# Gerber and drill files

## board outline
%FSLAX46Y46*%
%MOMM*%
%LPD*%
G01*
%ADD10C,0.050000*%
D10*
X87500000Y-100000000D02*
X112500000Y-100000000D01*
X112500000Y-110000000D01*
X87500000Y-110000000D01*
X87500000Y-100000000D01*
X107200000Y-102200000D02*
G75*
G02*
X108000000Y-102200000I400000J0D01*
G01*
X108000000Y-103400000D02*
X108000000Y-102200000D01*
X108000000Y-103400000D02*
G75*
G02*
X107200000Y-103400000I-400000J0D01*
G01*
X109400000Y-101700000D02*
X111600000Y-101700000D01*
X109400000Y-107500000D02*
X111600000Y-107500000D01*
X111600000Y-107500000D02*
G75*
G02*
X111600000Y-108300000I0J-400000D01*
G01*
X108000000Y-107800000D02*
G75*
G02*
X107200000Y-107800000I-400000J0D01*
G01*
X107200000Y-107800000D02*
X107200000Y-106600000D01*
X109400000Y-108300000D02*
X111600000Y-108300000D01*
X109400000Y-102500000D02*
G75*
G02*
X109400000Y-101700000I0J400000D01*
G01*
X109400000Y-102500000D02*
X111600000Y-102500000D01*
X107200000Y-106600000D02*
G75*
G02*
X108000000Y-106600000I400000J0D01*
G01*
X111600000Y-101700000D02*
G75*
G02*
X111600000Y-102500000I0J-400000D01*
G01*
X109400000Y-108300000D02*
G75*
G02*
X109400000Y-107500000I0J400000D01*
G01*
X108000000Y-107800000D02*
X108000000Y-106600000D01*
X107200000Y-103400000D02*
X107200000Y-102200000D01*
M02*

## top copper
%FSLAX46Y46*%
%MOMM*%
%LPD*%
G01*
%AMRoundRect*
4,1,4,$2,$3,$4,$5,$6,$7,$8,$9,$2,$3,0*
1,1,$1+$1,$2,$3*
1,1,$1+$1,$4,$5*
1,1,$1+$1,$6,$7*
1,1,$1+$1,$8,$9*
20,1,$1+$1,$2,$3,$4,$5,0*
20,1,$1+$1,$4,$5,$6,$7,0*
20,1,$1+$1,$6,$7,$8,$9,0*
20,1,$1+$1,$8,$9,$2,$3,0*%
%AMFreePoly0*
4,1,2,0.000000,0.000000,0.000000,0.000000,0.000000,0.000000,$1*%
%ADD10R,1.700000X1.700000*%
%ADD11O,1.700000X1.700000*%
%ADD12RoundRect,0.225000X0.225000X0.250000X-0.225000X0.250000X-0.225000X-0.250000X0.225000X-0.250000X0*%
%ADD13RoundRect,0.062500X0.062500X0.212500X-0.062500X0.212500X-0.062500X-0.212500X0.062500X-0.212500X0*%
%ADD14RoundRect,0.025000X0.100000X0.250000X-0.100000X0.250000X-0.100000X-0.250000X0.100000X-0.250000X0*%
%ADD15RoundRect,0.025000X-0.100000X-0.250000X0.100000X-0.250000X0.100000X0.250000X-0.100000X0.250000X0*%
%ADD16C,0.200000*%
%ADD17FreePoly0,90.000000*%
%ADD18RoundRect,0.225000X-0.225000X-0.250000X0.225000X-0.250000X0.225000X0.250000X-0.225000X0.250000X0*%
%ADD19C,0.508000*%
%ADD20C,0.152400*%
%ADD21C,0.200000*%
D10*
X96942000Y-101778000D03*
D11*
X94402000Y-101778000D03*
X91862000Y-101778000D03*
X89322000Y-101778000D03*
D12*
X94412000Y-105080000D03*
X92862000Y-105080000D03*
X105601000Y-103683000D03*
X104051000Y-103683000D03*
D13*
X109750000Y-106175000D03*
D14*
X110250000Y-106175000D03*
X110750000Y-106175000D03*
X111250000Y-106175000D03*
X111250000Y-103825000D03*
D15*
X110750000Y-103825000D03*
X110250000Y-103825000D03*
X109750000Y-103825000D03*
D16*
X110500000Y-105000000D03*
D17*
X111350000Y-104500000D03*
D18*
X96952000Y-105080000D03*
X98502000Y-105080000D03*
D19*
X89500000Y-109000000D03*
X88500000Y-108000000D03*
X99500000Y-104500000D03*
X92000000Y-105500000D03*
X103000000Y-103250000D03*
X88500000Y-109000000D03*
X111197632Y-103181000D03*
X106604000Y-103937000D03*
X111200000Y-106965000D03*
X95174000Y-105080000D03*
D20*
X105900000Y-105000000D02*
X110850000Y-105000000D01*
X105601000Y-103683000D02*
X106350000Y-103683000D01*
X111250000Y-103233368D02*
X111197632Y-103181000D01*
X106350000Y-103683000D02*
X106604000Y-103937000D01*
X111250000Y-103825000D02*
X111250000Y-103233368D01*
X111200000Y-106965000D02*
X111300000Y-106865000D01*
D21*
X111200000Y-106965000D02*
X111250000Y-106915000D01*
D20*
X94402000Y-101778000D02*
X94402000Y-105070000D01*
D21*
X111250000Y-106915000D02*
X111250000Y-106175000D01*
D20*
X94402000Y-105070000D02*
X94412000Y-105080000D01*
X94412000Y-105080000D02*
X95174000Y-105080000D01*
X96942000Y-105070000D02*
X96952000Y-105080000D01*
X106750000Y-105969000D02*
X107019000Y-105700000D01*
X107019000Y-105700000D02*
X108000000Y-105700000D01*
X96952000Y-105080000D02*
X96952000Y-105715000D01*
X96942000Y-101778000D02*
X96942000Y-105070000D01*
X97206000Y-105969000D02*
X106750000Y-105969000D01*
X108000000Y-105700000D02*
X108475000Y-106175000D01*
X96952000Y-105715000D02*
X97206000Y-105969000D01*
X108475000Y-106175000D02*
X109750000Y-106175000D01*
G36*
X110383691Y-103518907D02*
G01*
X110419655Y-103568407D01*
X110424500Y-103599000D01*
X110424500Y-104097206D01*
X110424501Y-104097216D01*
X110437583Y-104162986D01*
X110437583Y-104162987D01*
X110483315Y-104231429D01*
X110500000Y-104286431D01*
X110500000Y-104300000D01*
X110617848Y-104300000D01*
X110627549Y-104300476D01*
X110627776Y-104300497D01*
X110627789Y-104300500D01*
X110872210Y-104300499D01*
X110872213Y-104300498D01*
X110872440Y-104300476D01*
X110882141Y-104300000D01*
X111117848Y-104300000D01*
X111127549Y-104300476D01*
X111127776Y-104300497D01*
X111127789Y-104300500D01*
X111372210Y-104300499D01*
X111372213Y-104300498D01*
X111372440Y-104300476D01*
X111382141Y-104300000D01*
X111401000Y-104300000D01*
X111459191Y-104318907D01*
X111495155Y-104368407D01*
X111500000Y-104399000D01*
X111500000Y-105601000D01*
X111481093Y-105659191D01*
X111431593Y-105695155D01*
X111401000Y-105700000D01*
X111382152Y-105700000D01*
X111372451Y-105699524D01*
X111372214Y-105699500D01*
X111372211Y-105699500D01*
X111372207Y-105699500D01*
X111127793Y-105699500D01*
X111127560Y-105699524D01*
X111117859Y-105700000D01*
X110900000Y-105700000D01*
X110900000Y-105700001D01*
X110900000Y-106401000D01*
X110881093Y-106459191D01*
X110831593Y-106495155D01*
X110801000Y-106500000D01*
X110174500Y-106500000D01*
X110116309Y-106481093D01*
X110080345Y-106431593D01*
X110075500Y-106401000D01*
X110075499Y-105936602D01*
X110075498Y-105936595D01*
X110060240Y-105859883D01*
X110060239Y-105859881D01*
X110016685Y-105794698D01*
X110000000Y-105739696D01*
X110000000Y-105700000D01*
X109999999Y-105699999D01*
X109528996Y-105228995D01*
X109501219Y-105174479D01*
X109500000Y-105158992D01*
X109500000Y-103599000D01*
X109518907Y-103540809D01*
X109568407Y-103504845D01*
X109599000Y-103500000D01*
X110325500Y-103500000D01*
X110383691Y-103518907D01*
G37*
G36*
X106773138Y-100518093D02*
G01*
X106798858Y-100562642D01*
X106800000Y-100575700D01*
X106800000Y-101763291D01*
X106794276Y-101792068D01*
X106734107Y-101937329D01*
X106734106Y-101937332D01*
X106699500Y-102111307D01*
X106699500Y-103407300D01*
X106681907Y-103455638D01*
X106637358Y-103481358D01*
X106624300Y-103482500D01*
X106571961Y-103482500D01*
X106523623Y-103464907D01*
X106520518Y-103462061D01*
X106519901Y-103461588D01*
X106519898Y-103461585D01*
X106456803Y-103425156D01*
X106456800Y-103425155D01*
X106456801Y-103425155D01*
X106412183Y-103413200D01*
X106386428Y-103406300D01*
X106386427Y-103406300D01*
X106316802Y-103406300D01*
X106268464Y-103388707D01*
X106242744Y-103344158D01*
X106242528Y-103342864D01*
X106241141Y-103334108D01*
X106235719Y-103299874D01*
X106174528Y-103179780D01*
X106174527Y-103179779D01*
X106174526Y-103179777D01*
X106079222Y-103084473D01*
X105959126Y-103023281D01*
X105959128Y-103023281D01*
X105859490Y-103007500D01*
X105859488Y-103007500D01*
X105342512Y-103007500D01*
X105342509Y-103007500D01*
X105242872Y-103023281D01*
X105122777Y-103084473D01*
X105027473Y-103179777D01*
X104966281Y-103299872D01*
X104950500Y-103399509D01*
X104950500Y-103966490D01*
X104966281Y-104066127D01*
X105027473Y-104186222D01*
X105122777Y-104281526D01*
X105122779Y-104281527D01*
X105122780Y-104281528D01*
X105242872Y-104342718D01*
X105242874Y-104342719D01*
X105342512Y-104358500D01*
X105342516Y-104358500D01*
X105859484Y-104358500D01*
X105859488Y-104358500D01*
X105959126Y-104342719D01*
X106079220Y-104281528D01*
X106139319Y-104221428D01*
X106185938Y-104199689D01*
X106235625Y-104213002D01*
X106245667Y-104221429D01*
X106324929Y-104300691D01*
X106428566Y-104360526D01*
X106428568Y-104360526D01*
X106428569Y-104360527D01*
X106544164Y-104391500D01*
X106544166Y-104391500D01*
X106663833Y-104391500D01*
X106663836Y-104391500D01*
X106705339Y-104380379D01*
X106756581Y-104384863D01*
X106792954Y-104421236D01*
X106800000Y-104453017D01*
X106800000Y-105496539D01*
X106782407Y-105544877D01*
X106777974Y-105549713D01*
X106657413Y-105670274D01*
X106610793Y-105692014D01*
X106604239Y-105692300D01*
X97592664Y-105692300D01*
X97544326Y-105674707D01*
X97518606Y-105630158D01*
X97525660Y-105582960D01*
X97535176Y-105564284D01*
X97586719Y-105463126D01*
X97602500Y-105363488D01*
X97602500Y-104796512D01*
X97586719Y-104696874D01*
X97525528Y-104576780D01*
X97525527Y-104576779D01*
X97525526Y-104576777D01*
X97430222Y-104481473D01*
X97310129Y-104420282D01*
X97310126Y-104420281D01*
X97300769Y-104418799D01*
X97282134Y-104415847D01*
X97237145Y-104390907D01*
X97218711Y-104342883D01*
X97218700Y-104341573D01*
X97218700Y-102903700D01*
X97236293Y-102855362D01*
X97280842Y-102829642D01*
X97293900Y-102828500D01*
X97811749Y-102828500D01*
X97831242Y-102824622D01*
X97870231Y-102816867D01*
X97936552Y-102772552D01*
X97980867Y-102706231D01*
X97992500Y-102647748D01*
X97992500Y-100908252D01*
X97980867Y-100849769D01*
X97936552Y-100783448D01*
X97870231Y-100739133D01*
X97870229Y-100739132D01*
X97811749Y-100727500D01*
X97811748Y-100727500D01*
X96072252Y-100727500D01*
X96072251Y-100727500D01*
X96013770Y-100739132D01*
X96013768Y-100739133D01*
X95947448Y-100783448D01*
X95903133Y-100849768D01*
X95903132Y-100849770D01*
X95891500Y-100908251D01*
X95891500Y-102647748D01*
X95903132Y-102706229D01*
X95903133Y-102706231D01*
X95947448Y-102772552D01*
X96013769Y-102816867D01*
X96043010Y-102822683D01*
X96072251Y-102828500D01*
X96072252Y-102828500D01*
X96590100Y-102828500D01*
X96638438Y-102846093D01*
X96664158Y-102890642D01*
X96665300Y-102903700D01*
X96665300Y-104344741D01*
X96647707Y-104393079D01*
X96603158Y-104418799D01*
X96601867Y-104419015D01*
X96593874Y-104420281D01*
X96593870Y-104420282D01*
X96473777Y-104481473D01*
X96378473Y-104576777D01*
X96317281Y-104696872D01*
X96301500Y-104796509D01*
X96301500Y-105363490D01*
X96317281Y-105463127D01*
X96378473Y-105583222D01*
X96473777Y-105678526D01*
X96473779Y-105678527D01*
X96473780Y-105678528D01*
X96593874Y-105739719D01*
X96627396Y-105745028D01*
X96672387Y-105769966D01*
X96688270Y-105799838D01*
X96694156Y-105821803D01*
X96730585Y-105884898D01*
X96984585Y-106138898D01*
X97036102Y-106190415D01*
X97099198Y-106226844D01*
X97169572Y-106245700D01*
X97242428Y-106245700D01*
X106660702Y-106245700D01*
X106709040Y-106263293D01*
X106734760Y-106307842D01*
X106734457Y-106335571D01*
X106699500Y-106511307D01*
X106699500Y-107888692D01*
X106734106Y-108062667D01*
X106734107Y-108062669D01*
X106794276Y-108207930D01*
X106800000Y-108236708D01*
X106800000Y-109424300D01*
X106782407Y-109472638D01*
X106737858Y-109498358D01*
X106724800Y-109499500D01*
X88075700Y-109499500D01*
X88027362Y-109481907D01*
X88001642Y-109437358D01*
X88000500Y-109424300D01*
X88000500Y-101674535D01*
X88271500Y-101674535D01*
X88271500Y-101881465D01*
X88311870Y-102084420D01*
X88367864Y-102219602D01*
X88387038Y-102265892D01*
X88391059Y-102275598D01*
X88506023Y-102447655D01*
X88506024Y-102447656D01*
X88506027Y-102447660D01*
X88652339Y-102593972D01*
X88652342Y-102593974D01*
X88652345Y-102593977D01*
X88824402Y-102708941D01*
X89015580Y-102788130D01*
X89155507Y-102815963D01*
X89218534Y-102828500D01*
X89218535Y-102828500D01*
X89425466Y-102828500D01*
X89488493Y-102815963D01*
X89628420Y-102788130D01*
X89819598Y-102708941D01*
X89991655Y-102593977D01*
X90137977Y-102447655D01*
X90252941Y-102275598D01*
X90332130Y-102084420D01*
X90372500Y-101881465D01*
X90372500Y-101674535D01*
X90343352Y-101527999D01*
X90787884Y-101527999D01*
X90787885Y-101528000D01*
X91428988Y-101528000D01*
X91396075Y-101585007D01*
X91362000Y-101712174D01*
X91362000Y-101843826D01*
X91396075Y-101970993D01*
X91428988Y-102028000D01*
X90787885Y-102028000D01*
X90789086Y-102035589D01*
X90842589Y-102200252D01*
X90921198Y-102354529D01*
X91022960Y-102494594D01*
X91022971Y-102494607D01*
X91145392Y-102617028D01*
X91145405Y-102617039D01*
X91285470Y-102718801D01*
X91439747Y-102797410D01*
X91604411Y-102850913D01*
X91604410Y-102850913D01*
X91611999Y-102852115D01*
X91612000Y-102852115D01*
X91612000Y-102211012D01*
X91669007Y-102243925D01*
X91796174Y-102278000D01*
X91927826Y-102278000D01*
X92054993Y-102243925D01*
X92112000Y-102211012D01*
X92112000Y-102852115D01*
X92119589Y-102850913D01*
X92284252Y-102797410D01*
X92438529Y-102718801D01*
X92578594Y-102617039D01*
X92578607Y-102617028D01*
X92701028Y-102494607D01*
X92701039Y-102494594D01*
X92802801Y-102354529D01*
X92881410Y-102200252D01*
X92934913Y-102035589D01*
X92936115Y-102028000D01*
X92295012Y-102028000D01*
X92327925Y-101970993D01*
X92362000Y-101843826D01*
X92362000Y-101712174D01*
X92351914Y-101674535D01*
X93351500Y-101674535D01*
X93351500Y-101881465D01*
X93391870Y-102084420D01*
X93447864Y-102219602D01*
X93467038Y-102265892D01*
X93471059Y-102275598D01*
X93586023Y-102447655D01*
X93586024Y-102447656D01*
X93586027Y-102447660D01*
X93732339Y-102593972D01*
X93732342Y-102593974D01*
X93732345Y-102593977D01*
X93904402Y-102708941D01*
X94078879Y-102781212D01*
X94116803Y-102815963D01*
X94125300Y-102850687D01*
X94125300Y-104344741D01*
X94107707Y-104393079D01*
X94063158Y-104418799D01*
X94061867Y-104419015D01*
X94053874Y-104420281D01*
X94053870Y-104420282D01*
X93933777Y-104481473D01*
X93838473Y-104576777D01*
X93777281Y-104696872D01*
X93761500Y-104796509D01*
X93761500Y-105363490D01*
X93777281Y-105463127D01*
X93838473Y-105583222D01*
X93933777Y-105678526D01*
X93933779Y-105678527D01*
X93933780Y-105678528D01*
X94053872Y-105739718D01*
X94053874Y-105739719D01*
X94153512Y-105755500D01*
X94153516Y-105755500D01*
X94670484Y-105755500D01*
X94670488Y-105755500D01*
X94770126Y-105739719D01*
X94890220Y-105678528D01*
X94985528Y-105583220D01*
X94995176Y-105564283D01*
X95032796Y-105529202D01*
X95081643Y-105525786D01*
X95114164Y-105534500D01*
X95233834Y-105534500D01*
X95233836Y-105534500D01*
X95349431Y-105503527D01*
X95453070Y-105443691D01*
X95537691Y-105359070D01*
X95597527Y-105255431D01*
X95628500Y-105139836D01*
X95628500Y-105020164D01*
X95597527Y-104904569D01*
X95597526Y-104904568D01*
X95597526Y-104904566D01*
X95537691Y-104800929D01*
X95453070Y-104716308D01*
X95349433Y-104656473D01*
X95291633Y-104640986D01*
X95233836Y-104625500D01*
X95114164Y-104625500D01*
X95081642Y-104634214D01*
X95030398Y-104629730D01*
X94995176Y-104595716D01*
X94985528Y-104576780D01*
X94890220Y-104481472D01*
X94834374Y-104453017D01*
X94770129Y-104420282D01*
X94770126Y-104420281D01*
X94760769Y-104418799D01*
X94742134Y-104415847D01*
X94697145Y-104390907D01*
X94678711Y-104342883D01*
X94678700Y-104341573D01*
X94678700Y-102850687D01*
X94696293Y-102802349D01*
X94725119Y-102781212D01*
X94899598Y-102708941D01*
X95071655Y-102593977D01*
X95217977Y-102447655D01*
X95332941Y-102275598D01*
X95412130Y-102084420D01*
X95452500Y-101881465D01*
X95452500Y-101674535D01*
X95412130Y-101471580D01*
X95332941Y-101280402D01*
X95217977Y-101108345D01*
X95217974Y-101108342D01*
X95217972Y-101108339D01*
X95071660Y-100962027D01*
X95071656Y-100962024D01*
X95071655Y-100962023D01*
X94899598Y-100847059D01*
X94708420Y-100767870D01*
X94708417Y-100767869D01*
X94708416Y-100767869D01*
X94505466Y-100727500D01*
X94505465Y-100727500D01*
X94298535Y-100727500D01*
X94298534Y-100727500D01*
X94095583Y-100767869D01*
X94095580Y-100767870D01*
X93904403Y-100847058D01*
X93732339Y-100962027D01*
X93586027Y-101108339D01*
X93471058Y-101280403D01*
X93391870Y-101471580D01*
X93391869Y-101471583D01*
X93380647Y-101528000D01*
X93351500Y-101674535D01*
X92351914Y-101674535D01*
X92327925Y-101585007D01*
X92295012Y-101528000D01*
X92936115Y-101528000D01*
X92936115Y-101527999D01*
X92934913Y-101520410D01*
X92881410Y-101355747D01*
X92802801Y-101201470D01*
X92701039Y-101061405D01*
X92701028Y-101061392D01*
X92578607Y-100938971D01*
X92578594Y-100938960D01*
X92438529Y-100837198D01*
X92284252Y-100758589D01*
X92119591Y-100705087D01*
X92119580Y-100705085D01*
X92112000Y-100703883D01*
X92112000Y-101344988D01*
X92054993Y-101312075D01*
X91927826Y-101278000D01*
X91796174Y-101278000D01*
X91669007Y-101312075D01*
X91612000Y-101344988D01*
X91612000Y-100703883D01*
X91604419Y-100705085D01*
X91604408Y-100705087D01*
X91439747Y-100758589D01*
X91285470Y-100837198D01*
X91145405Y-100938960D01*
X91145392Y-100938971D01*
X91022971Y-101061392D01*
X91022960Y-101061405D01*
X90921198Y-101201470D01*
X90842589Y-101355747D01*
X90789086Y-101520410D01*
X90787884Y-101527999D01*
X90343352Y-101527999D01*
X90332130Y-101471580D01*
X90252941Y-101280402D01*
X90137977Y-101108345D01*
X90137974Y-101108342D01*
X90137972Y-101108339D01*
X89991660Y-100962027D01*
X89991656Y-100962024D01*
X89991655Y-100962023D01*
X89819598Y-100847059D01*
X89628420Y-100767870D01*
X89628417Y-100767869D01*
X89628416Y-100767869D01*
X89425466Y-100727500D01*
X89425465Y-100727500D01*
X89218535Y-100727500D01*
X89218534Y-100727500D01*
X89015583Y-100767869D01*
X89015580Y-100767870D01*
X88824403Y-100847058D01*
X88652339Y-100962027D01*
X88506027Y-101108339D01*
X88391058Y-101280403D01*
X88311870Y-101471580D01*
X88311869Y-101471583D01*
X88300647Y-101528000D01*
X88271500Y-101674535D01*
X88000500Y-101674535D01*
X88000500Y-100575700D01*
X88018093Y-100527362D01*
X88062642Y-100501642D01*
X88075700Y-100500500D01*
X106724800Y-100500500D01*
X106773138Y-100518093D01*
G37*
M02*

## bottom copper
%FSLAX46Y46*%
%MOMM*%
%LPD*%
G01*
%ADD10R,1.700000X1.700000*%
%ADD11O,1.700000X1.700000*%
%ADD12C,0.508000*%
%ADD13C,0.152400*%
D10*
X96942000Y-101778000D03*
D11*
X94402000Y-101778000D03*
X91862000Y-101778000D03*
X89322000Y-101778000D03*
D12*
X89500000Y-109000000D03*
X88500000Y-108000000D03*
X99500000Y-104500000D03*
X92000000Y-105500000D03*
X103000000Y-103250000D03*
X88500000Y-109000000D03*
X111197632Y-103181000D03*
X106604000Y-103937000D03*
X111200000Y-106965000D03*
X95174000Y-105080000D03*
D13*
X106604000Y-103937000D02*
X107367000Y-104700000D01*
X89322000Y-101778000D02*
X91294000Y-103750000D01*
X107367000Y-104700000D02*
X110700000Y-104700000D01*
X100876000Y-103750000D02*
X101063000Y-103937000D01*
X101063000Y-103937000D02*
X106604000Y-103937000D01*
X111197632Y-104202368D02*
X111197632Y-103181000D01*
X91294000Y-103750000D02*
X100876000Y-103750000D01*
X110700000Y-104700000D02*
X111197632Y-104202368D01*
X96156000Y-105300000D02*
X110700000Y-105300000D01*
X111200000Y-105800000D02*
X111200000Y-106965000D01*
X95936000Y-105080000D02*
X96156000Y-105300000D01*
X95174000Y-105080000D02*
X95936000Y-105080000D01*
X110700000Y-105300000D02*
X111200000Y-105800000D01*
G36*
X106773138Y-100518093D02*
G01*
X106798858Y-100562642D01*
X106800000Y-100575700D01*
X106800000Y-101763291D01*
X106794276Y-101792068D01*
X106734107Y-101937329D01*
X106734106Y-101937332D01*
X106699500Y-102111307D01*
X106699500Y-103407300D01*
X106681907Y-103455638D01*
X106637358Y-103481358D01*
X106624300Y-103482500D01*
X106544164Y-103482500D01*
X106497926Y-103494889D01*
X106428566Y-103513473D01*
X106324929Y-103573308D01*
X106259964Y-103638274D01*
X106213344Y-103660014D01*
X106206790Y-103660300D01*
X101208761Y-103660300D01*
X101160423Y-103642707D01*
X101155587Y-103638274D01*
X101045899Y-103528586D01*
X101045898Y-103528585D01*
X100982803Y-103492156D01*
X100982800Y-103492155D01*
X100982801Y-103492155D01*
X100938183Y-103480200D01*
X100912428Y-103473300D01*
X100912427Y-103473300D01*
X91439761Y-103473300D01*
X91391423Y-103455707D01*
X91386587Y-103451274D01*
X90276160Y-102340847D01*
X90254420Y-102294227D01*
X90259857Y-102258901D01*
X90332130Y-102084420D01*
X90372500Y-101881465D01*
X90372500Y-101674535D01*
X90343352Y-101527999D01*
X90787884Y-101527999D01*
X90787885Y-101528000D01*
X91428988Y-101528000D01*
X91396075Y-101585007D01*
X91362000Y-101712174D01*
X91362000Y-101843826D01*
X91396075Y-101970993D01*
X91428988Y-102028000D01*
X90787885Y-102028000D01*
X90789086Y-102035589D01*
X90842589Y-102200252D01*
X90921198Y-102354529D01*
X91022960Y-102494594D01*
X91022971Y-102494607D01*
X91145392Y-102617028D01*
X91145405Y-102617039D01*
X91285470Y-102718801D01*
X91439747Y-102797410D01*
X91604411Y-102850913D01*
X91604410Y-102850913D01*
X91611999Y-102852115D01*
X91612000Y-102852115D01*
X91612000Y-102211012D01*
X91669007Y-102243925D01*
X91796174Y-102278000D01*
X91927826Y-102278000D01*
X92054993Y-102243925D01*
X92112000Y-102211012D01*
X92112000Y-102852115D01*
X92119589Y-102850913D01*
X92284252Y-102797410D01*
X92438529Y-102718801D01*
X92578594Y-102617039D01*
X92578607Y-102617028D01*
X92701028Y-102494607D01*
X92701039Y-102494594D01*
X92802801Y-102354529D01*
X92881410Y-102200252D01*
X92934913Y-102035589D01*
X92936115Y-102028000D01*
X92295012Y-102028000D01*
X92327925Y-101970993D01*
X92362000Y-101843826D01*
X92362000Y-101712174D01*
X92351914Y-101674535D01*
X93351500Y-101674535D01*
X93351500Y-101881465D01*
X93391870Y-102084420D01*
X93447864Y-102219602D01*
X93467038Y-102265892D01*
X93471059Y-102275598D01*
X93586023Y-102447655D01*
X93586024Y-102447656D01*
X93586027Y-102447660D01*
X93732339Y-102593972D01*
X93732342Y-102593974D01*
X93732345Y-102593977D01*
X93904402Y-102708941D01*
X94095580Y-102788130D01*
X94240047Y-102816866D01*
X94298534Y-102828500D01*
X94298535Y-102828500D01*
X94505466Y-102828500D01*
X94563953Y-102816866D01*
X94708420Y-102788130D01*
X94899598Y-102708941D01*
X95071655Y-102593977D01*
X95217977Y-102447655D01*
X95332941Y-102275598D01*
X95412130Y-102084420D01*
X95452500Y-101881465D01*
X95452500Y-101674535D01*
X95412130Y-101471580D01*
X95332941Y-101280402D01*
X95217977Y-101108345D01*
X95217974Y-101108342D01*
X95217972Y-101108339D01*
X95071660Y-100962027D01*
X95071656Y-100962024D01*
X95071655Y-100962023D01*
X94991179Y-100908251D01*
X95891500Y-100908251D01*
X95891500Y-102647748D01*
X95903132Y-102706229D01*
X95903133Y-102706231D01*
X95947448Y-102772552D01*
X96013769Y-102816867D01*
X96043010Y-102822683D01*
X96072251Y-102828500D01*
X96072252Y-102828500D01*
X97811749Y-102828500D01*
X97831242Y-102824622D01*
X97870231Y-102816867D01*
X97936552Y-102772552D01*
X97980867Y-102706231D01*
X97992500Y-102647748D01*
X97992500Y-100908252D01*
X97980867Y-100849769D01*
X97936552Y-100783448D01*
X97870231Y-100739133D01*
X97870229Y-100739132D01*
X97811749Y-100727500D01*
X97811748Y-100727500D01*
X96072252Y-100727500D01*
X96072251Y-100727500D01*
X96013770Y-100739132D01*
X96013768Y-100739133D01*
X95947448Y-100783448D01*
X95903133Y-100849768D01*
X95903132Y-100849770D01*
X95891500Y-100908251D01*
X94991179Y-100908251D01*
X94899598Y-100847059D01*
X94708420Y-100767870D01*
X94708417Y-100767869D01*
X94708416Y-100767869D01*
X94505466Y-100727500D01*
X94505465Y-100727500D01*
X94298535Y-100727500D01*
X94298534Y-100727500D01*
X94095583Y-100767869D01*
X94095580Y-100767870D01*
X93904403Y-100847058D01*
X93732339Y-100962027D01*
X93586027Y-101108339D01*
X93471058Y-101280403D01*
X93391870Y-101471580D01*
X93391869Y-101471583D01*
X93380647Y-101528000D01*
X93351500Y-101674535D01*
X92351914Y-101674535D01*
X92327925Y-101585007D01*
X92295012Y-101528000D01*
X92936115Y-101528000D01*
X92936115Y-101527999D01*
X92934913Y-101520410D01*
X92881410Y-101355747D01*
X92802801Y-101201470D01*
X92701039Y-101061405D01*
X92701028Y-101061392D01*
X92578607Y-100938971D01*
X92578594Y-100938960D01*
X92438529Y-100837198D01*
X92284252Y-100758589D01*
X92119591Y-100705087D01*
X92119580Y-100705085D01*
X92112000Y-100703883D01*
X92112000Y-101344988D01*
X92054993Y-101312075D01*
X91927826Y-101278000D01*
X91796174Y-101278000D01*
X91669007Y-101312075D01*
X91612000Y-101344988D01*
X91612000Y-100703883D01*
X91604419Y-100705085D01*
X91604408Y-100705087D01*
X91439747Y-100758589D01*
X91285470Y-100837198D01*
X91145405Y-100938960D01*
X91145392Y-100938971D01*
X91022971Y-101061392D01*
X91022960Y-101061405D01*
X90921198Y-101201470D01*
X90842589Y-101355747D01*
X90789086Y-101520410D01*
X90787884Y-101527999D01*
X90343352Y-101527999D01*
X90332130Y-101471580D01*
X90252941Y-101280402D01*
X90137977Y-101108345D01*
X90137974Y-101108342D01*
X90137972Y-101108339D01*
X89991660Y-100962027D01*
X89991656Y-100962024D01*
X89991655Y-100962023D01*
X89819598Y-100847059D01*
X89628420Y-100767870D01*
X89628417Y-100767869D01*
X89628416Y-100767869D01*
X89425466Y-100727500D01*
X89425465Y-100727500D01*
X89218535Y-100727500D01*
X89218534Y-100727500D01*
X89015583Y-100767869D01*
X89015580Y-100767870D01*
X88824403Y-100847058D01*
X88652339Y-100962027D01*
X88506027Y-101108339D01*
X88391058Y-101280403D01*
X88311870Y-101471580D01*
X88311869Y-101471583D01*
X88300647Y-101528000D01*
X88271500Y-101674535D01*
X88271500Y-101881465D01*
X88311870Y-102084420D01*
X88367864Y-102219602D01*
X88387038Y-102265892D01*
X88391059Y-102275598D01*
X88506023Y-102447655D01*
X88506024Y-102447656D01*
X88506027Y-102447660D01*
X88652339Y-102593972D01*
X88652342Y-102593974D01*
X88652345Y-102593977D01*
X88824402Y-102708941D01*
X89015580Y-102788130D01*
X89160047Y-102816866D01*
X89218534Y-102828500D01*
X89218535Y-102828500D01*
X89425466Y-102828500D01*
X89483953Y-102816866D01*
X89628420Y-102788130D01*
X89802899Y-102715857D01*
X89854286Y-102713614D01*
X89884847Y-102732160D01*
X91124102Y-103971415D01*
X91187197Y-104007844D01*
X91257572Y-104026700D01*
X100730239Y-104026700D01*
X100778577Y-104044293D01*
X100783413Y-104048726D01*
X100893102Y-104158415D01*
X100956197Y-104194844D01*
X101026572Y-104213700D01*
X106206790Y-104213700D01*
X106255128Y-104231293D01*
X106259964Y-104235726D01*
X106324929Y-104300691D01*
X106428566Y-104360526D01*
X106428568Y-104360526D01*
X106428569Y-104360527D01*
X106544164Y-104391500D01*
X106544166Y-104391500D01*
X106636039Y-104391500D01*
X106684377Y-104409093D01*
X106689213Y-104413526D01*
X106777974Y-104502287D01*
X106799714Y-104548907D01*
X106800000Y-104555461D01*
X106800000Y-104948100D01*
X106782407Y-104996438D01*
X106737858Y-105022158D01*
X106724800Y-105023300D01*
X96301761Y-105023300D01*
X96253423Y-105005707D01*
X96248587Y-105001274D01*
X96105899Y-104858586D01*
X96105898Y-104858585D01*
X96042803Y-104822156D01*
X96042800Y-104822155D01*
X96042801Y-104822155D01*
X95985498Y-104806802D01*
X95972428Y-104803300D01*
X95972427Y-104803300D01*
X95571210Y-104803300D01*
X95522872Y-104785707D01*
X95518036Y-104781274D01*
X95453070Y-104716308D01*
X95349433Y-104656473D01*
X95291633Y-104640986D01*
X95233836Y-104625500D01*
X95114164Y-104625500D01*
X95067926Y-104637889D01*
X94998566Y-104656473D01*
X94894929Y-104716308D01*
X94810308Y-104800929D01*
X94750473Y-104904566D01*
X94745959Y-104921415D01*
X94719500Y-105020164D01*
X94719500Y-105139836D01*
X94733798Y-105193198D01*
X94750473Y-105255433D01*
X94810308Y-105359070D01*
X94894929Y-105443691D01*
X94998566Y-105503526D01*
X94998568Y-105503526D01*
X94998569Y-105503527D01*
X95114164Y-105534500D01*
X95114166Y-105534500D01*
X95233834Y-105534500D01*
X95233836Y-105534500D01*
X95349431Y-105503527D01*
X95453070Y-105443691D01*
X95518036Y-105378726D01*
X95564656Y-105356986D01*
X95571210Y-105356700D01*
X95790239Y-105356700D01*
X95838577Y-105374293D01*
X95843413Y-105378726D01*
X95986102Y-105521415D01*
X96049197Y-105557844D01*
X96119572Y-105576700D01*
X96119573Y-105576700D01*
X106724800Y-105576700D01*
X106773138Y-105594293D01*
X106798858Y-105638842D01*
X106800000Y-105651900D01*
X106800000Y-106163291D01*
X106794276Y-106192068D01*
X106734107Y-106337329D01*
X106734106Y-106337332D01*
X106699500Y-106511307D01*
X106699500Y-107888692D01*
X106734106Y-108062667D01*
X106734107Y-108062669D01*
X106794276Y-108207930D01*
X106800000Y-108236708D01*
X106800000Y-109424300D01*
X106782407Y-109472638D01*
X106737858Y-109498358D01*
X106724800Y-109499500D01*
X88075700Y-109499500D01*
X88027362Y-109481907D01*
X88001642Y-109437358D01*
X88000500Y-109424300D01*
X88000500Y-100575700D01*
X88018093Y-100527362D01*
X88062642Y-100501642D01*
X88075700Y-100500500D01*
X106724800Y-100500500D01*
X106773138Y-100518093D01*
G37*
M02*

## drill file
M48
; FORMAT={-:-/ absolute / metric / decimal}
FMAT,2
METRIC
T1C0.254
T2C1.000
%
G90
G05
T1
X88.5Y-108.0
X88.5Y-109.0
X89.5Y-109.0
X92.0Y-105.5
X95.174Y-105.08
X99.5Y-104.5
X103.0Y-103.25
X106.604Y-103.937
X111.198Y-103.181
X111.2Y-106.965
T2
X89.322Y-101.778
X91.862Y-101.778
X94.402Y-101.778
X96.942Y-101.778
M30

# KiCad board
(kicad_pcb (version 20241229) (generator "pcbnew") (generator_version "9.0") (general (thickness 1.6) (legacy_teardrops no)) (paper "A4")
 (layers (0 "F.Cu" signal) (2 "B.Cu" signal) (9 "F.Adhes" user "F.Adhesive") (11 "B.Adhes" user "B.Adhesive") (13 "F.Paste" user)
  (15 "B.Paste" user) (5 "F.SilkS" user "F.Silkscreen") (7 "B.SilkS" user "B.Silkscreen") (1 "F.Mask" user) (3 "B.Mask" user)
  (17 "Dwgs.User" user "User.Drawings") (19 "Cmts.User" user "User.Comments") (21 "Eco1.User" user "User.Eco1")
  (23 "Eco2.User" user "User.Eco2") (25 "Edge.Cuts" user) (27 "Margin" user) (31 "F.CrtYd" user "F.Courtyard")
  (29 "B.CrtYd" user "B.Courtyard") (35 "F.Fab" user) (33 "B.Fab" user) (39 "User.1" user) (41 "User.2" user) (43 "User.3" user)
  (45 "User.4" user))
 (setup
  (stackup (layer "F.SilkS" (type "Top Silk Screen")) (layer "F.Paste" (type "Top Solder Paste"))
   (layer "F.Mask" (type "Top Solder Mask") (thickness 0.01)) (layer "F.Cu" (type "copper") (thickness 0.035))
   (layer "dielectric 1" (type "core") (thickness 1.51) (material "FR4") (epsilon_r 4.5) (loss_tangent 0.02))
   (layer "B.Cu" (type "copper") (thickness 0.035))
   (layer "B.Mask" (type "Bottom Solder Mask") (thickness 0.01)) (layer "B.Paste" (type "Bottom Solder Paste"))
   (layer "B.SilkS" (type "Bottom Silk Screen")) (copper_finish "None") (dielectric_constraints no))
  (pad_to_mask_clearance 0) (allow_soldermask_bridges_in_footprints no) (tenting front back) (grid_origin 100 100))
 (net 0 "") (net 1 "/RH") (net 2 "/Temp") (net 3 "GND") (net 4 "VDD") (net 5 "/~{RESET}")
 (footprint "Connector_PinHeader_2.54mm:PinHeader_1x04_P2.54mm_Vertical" (layer "F.Cu") (at 96.942 101.778 -90)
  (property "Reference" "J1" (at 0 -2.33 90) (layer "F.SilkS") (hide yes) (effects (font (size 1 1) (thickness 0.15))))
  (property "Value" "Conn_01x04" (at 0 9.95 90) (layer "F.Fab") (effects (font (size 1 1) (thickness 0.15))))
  (pad "1" thru_hole rect (at 0 0 270) (size 1.7 1.7) (drill 1) (layers "*.Cu" "*.Mask") (remove_unused_layers no) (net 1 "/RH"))
  (pad "2" thru_hole oval (at 0 2.54 270) (size 1.7 1.7) (drill 1) (layers "*.Cu" "*.Mask") (remove_unused_layers no) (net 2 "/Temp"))
  (pad "3" thru_hole oval (at 0 5.08 270) (size 1.7 1.7) (drill 1) (layers "*.Cu" "*.Mask") (remove_unused_layers no) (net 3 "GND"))
  (pad "4" thru_hole oval (at 0 7.62 270) (size 1.7 1.7) (drill 1) (layers "*.Cu" "*.Mask") (remove_unused_layers no) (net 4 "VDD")))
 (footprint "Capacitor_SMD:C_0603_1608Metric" (layer "F.Cu") (at 93.637 105.08 180)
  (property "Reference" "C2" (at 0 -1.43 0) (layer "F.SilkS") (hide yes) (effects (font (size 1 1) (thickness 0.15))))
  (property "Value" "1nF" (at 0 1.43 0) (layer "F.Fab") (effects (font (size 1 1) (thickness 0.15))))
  (pad "1" smd roundrect (at -0.775 0 180) (size 0.9 0.95) (layers "F.Cu" "F.Mask" "F.Paste") (roundrect_rratio 0.25) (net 2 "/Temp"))
  (pad "2" smd roundrect (at 0.775 0 180) (size 0.9 0.95) (layers "F.Cu" "F.Mask" "F.Paste") (roundrect_rratio 0.25) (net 3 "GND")))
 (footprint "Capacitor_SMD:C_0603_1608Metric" (layer "F.Cu") (at 104.826 103.683 180)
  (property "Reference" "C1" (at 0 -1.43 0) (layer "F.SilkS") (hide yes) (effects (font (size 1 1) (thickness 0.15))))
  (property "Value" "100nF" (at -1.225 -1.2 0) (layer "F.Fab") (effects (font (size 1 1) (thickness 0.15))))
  (pad "1" smd roundrect (at -0.775 0 180) (size 0.9 0.95) (layers "F.Cu" "F.Mask" "F.Paste") (roundrect_rratio 0.25) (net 4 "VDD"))
  (pad "2" smd roundrect (at 0.775 0 180) (size 0.9 0.95) (layers "F.Cu" "F.Mask" "F.Paste") (roundrect_rratio 0.25) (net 3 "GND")))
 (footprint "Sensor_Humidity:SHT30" (layer "F.Cu") (at 110.5 105 90)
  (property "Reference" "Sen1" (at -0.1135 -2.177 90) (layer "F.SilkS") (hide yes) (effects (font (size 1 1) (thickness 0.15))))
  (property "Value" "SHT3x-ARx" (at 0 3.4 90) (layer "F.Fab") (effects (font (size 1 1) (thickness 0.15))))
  (pad "1" smd roundrect (at -1.175 -0.75 180) (size 0.25 0.55) (layers "F.Cu" "F.Mask" "F.Paste") (roundrect_rratio 0.25) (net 1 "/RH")
   (solder_mask_margin 0.05) (solder_paste_margin 0))
  (pad "2" smd roundrect (at -1.175 -0.25 180) (size 0.25 0.55) (layers "F.Cu" "F.Mask" "F.Paste") (roundrect_rratio 0.1) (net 3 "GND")
   (solder_mask_margin 0.05) (solder_paste_margin 0))
  (pad "3" smd roundrect (at -1.175 0.25 180) (size 0.25 0.55) (layers "F.Cu" "F.Mask" "F.Paste") (roundrect_rratio 0.1) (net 3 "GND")
   (solder_mask_margin 0.05) (solder_paste_margin 0))
  (pad "4" smd roundrect (at -1.175 0.75 180) (size 0.25 0.55) (layers "F.Cu" "F.Mask" "F.Paste") (roundrect_rratio 0.1) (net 2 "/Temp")
   (solder_mask_margin 0.05) (solder_paste_margin 0))
  (pad "5" smd roundrect (at 1.175 0.75 180) (size 0.25 0.55) (layers "F.Cu" "F.Mask" "F.Paste") (roundrect_rratio 0.1) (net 4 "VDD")
   (solder_mask_margin 0.05) (solder_paste_margin 0))
  (pad "6" smd roundrect (at 1.175 0.25) (size 0.25 0.55) (layers "F.Cu" "F.Mask" "F.Paste") (roundrect_rratio 0.1) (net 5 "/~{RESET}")
   (solder_mask_margin 0.05) (solder_paste_margin 0))
  (pad "7" smd roundrect (at 1.175 -0.25) (size 0.25 0.55) (layers "F.Cu" "F.Mask" "F.Paste") (roundrect_rratio 0.1) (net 3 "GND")
   (solder_mask_margin 0.05) (solder_paste_margin 0))
  (pad "8" smd roundrect (at 1.175 -0.75) (size 0.25 0.55) (layers "F.Cu" "F.Mask" "F.Paste") (roundrect_rratio 0.1) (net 3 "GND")
   (solder_mask_margin 0.05) (solder_paste_margin 0))
  (pad "9" smd circle (at 0 0 270) (size 0.2 0.2) (layers "F.Cu" "F.Mask" "F.Paste") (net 3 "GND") (solder_mask_margin 0.05)
   (thermal_bridge_angle 90))
  (pad "9" smd custom (at 0.5 0.85 90) (size 0.000001 0.000001) (layers "F.Cu" "F.Mask" "F.Paste") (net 3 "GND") (solder_mask_margin 0.05)
   (solder_paste_margin -0.1) (thermal_bridge_angle 90) (options (clearance outline) (anchor circle)) (primitives)))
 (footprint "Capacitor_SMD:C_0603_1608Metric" (layer "F.Cu") (at 97.727 105.08)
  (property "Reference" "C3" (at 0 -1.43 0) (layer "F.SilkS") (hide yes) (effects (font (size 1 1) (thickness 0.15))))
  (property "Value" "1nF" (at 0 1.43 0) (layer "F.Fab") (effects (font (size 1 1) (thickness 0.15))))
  (pad "1" smd roundrect (at -0.775 0) (size 0.9 0.95) (layers "F.Cu" "F.Mask" "F.Paste") (roundrect_rratio 0.25) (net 1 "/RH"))
  (pad "2" smd roundrect (at 0.775 0) (size 0.9 0.95) (layers "F.Cu" "F.Mask" "F.Paste") (roundrect_rratio 0.25) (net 3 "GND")))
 (gr_rect (start 87.5 100) (end 112.5 110) (stroke (width 0.05) (type default)) (fill no) (layer "Edge.Cuts"))
 (gr_arc (start 107.2 102.2) (mid 107.6 101.8) (end 108 102.2) (stroke (width 0.05) (type default)) (layer "Edge.Cuts"))
 (gr_line (start 108 103.4) (end 108 102.2) (stroke (width 0.05) (type default)) (layer "Edge.Cuts"))
 (gr_arc (start 108 103.4) (mid 107.6 103.8) (end 107.2 103.4) (stroke (width 0.05) (type default)) (layer "Edge.Cuts"))
 (gr_line (start 109.4 101.7) (end 111.6 101.7) (stroke (width 0.05) (type default)) (layer "Edge.Cuts"))
 (gr_line (start 109.4 107.5) (end 111.6 107.5) (stroke (width 0.05) (type default)) (layer "Edge.Cuts"))
 (gr_arc (start 111.6 107.5) (mid 112 107.9) (end 111.6 108.3) (stroke (width 0.05) (type default)) (layer "Edge.Cuts"))
 (gr_arc (start 108 107.8) (mid 107.6 108.2) (end 107.2 107.8) (stroke (width 0.05) (type default)) (layer "Edge.Cuts"))
 (gr_line (start 107.2 107.8) (end 107.2 106.6) (stroke (width 0.05) (type default)) (layer "Edge.Cuts"))
 (gr_line (start 109.4 108.3) (end 111.6 108.3) (stroke (width 0.05) (type default)) (layer "Edge.Cuts"))
 (gr_arc (start 109.4 102.5) (mid 109 102.1) (end 109.4 101.7) (stroke (width 0.05) (type default)) (layer "Edge.Cuts"))
 (gr_line (start 109.4 102.5) (end 111.6 102.5) (stroke (width 0.05) (type default)) (layer "Edge.Cuts"))
 (gr_arc (start 107.2 106.6) (mid 107.6 106.2) (end 108 106.6) (stroke (width 0.05) (type default)) (layer "Edge.Cuts"))
 (gr_arc (start 111.6 101.7) (mid 112 102.1) (end 111.6 102.5) (stroke (width 0.05) (type default)) (layer "Edge.Cuts"))
 (gr_arc (start 109.4 108.3) (mid 109 107.9) (end 109.4 107.5) (stroke (width 0.05) (type default)) (layer "Edge.Cuts"))
 (gr_line (start 108 107.8) (end 108 106.6) (stroke (width 0.05) (type default)) (layer "Edge.Cuts"))
 (gr_line (start 107.2 103.4) (end 107.2 102.2) (stroke (width 0.05) (type default)) (layer "Edge.Cuts"))
 (segment (start 105.9 105) (end 110.85 105) (width 0.1524) (layer "F.Cu") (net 3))
 (via (at 89.5 109) (size 0.508) (drill 0.254) (layers "F.Cu" "B.Cu") (free yes) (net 3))
 (via (at 88.5 108) (size 0.508) (drill 0.254) (layers "F.Cu" "B.Cu") (free yes) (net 3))
 (via (at 99.5 104.5) (size 0.508) (drill 0.254) (layers "F.Cu" "B.Cu") (free yes) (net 3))
 (via (at 92 105.5) (size 0.508) (drill 0.254) (layers "F.Cu" "B.Cu") (free yes) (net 3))
 (via (at 103 103.25) (size 0.508) (drill 0.254) (layers "F.Cu" "B.Cu") (free yes) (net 3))
 (via (at 88.5 109) (size 0.508) (drill 0.254) (layers "F.Cu" "B.Cu") (free yes) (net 3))
 (segment (start 105.601 103.683) (end 106.35 103.683) (width 0.1524) (layer "F.Cu") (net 4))
 (segment (start 111.25 103.233368) (end 111.197632 103.181) (width 0.1524) (layer "F.Cu") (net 4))
 (segment (start 106.35 103.683) (end 106.604 103.937) (width 0.1524) (layer "F.Cu") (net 4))
 (segment (start 111.25 103.825) (end 111.25 103.233368) (width 0.1524) (layer "F.Cu") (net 4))
 (via (at 111.197632 103.181) (size 0.508) (drill 0.254) (layers "F.Cu" "B.Cu") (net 4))
 (via (at 106.604 103.937) (size 0.508) (drill 0.254) (layers "F.Cu" "B.Cu") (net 4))
 (segment (start 106.604 103.937) (end 107.367 104.7) (width 0.1524) (layer "B.Cu") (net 4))
 (segment (start 89.322 101.778) (end 91.294 103.75) (width 0.1524) (layer "B.Cu") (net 4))
 (segment (start 107.367 104.7) (end 110.7 104.7) (width 0.1524) (layer "B.Cu") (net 4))
 (segment (start 100.876 103.75) (end 101.063 103.937) (width 0.1524) (layer "B.Cu") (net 4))
 (segment (start 101.063 103.937) (end 106.604 103.937) (width 0.1524) (layer "B.Cu") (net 4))
 (segment (start 111.197632 104.202368) (end 111.197632 103.181) (width 0.1524) (layer "B.Cu") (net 4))
 (segment (start 91.294 103.75) (end 100.876 103.75) (width 0.1524) (layer "B.Cu") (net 4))
 (segment (start 110.7 104.7) (end 111.197632 104.202368) (width 0.1524) (layer "B.Cu") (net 4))
 (segment (start 111.2 106.965) (end 111.3 106.865) (width 0.1524) (layer "F.Cu") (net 2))
 (segment (start 111.2 106.965) (end 111.25 106.915) (width 0.2) (layer "F.Cu") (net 2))
 (segment (start 94.402 101.778) (end 94.402 105.07) (width 0.1524) (layer "F.Cu") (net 2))
 (segment (start 111.25 106.915) (end 111.25 106.175) (width 0.2) (layer "F.Cu") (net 2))
 (segment (start 94.402 105.07) (end 94.412 105.08) (width 0.1524) (layer "F.Cu") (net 2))
 (segment (start 94.412 105.08) (end 95.174 105.08) (width 0.1524) (layer "F.Cu") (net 2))
 (via (at 111.2 106.965) (size 0.508) (drill 0.254) (layers "F.Cu" "B.Cu") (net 2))
 (via (at 95.174 105.08) (size 0.508) (drill 0.254) (layers "F.Cu" "B.Cu") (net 2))
 (segment (start 96.156 105.3) (end 110.7 105.3) (width 0.1524) (layer "B.Cu") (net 2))
 (segment (start 111.2 105.8) (end 111.2 106.965) (width 0.1524) (layer "B.Cu") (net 2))
 (segment (start 95.936 105.08) (end 96.156 105.3) (width 0.1524) (layer "B.Cu") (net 2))
 (segment (start 95.174 105.08) (end 95.936 105.08) (width 0.1524) (layer "B.Cu") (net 2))
 (segment (start 110.7 105.3) (end 111.2 105.8) (width 0.1524) (layer "B.Cu") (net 2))
 (segment (start 96.942 105.07) (end 96.952 105.08) (width 0.1524) (layer "F.Cu") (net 1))
 (segment (start 106.75 105.969) (end 107.019 105.7) (width 0.1524) (layer "F.Cu") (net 1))
 (segment (start 107.019 105.7) (end 108 105.7) (width 0.1524) (layer "F.Cu") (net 1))
 (segment (start 96.952 105.08) (end 96.952 105.715) (width 0.1524) (layer "F.Cu") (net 1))
 (segment (start 96.942 101.778) (end 96.942 105.07) (width 0.1524) (layer "F.Cu") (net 1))
 (segment (start 97.206 105.969) (end 106.75 105.969) (width 0.1524) (layer "F.Cu") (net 1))
 (segment (start 108 105.7) (end 108.475 106.175) (width 0.1524) (layer "F.Cu") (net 1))
 (segment (start 96.952 105.715) (end 97.206 105.969) (width 0.1524) (layer "F.Cu") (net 1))
 (segment (start 108.475 106.175) (end 109.75 106.175) (width 0.1524) (layer "F.Cu") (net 1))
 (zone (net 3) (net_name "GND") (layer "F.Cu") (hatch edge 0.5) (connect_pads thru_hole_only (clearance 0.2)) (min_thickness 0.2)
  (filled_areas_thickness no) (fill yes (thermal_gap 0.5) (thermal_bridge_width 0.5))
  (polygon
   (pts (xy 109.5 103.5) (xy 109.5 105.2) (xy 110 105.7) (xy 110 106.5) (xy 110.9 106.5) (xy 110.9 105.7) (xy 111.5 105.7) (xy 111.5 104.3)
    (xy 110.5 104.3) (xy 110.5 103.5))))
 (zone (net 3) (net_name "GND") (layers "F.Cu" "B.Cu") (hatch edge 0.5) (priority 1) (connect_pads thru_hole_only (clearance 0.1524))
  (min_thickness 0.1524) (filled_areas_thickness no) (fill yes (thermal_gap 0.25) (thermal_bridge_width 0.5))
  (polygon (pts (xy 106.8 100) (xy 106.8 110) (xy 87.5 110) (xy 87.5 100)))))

